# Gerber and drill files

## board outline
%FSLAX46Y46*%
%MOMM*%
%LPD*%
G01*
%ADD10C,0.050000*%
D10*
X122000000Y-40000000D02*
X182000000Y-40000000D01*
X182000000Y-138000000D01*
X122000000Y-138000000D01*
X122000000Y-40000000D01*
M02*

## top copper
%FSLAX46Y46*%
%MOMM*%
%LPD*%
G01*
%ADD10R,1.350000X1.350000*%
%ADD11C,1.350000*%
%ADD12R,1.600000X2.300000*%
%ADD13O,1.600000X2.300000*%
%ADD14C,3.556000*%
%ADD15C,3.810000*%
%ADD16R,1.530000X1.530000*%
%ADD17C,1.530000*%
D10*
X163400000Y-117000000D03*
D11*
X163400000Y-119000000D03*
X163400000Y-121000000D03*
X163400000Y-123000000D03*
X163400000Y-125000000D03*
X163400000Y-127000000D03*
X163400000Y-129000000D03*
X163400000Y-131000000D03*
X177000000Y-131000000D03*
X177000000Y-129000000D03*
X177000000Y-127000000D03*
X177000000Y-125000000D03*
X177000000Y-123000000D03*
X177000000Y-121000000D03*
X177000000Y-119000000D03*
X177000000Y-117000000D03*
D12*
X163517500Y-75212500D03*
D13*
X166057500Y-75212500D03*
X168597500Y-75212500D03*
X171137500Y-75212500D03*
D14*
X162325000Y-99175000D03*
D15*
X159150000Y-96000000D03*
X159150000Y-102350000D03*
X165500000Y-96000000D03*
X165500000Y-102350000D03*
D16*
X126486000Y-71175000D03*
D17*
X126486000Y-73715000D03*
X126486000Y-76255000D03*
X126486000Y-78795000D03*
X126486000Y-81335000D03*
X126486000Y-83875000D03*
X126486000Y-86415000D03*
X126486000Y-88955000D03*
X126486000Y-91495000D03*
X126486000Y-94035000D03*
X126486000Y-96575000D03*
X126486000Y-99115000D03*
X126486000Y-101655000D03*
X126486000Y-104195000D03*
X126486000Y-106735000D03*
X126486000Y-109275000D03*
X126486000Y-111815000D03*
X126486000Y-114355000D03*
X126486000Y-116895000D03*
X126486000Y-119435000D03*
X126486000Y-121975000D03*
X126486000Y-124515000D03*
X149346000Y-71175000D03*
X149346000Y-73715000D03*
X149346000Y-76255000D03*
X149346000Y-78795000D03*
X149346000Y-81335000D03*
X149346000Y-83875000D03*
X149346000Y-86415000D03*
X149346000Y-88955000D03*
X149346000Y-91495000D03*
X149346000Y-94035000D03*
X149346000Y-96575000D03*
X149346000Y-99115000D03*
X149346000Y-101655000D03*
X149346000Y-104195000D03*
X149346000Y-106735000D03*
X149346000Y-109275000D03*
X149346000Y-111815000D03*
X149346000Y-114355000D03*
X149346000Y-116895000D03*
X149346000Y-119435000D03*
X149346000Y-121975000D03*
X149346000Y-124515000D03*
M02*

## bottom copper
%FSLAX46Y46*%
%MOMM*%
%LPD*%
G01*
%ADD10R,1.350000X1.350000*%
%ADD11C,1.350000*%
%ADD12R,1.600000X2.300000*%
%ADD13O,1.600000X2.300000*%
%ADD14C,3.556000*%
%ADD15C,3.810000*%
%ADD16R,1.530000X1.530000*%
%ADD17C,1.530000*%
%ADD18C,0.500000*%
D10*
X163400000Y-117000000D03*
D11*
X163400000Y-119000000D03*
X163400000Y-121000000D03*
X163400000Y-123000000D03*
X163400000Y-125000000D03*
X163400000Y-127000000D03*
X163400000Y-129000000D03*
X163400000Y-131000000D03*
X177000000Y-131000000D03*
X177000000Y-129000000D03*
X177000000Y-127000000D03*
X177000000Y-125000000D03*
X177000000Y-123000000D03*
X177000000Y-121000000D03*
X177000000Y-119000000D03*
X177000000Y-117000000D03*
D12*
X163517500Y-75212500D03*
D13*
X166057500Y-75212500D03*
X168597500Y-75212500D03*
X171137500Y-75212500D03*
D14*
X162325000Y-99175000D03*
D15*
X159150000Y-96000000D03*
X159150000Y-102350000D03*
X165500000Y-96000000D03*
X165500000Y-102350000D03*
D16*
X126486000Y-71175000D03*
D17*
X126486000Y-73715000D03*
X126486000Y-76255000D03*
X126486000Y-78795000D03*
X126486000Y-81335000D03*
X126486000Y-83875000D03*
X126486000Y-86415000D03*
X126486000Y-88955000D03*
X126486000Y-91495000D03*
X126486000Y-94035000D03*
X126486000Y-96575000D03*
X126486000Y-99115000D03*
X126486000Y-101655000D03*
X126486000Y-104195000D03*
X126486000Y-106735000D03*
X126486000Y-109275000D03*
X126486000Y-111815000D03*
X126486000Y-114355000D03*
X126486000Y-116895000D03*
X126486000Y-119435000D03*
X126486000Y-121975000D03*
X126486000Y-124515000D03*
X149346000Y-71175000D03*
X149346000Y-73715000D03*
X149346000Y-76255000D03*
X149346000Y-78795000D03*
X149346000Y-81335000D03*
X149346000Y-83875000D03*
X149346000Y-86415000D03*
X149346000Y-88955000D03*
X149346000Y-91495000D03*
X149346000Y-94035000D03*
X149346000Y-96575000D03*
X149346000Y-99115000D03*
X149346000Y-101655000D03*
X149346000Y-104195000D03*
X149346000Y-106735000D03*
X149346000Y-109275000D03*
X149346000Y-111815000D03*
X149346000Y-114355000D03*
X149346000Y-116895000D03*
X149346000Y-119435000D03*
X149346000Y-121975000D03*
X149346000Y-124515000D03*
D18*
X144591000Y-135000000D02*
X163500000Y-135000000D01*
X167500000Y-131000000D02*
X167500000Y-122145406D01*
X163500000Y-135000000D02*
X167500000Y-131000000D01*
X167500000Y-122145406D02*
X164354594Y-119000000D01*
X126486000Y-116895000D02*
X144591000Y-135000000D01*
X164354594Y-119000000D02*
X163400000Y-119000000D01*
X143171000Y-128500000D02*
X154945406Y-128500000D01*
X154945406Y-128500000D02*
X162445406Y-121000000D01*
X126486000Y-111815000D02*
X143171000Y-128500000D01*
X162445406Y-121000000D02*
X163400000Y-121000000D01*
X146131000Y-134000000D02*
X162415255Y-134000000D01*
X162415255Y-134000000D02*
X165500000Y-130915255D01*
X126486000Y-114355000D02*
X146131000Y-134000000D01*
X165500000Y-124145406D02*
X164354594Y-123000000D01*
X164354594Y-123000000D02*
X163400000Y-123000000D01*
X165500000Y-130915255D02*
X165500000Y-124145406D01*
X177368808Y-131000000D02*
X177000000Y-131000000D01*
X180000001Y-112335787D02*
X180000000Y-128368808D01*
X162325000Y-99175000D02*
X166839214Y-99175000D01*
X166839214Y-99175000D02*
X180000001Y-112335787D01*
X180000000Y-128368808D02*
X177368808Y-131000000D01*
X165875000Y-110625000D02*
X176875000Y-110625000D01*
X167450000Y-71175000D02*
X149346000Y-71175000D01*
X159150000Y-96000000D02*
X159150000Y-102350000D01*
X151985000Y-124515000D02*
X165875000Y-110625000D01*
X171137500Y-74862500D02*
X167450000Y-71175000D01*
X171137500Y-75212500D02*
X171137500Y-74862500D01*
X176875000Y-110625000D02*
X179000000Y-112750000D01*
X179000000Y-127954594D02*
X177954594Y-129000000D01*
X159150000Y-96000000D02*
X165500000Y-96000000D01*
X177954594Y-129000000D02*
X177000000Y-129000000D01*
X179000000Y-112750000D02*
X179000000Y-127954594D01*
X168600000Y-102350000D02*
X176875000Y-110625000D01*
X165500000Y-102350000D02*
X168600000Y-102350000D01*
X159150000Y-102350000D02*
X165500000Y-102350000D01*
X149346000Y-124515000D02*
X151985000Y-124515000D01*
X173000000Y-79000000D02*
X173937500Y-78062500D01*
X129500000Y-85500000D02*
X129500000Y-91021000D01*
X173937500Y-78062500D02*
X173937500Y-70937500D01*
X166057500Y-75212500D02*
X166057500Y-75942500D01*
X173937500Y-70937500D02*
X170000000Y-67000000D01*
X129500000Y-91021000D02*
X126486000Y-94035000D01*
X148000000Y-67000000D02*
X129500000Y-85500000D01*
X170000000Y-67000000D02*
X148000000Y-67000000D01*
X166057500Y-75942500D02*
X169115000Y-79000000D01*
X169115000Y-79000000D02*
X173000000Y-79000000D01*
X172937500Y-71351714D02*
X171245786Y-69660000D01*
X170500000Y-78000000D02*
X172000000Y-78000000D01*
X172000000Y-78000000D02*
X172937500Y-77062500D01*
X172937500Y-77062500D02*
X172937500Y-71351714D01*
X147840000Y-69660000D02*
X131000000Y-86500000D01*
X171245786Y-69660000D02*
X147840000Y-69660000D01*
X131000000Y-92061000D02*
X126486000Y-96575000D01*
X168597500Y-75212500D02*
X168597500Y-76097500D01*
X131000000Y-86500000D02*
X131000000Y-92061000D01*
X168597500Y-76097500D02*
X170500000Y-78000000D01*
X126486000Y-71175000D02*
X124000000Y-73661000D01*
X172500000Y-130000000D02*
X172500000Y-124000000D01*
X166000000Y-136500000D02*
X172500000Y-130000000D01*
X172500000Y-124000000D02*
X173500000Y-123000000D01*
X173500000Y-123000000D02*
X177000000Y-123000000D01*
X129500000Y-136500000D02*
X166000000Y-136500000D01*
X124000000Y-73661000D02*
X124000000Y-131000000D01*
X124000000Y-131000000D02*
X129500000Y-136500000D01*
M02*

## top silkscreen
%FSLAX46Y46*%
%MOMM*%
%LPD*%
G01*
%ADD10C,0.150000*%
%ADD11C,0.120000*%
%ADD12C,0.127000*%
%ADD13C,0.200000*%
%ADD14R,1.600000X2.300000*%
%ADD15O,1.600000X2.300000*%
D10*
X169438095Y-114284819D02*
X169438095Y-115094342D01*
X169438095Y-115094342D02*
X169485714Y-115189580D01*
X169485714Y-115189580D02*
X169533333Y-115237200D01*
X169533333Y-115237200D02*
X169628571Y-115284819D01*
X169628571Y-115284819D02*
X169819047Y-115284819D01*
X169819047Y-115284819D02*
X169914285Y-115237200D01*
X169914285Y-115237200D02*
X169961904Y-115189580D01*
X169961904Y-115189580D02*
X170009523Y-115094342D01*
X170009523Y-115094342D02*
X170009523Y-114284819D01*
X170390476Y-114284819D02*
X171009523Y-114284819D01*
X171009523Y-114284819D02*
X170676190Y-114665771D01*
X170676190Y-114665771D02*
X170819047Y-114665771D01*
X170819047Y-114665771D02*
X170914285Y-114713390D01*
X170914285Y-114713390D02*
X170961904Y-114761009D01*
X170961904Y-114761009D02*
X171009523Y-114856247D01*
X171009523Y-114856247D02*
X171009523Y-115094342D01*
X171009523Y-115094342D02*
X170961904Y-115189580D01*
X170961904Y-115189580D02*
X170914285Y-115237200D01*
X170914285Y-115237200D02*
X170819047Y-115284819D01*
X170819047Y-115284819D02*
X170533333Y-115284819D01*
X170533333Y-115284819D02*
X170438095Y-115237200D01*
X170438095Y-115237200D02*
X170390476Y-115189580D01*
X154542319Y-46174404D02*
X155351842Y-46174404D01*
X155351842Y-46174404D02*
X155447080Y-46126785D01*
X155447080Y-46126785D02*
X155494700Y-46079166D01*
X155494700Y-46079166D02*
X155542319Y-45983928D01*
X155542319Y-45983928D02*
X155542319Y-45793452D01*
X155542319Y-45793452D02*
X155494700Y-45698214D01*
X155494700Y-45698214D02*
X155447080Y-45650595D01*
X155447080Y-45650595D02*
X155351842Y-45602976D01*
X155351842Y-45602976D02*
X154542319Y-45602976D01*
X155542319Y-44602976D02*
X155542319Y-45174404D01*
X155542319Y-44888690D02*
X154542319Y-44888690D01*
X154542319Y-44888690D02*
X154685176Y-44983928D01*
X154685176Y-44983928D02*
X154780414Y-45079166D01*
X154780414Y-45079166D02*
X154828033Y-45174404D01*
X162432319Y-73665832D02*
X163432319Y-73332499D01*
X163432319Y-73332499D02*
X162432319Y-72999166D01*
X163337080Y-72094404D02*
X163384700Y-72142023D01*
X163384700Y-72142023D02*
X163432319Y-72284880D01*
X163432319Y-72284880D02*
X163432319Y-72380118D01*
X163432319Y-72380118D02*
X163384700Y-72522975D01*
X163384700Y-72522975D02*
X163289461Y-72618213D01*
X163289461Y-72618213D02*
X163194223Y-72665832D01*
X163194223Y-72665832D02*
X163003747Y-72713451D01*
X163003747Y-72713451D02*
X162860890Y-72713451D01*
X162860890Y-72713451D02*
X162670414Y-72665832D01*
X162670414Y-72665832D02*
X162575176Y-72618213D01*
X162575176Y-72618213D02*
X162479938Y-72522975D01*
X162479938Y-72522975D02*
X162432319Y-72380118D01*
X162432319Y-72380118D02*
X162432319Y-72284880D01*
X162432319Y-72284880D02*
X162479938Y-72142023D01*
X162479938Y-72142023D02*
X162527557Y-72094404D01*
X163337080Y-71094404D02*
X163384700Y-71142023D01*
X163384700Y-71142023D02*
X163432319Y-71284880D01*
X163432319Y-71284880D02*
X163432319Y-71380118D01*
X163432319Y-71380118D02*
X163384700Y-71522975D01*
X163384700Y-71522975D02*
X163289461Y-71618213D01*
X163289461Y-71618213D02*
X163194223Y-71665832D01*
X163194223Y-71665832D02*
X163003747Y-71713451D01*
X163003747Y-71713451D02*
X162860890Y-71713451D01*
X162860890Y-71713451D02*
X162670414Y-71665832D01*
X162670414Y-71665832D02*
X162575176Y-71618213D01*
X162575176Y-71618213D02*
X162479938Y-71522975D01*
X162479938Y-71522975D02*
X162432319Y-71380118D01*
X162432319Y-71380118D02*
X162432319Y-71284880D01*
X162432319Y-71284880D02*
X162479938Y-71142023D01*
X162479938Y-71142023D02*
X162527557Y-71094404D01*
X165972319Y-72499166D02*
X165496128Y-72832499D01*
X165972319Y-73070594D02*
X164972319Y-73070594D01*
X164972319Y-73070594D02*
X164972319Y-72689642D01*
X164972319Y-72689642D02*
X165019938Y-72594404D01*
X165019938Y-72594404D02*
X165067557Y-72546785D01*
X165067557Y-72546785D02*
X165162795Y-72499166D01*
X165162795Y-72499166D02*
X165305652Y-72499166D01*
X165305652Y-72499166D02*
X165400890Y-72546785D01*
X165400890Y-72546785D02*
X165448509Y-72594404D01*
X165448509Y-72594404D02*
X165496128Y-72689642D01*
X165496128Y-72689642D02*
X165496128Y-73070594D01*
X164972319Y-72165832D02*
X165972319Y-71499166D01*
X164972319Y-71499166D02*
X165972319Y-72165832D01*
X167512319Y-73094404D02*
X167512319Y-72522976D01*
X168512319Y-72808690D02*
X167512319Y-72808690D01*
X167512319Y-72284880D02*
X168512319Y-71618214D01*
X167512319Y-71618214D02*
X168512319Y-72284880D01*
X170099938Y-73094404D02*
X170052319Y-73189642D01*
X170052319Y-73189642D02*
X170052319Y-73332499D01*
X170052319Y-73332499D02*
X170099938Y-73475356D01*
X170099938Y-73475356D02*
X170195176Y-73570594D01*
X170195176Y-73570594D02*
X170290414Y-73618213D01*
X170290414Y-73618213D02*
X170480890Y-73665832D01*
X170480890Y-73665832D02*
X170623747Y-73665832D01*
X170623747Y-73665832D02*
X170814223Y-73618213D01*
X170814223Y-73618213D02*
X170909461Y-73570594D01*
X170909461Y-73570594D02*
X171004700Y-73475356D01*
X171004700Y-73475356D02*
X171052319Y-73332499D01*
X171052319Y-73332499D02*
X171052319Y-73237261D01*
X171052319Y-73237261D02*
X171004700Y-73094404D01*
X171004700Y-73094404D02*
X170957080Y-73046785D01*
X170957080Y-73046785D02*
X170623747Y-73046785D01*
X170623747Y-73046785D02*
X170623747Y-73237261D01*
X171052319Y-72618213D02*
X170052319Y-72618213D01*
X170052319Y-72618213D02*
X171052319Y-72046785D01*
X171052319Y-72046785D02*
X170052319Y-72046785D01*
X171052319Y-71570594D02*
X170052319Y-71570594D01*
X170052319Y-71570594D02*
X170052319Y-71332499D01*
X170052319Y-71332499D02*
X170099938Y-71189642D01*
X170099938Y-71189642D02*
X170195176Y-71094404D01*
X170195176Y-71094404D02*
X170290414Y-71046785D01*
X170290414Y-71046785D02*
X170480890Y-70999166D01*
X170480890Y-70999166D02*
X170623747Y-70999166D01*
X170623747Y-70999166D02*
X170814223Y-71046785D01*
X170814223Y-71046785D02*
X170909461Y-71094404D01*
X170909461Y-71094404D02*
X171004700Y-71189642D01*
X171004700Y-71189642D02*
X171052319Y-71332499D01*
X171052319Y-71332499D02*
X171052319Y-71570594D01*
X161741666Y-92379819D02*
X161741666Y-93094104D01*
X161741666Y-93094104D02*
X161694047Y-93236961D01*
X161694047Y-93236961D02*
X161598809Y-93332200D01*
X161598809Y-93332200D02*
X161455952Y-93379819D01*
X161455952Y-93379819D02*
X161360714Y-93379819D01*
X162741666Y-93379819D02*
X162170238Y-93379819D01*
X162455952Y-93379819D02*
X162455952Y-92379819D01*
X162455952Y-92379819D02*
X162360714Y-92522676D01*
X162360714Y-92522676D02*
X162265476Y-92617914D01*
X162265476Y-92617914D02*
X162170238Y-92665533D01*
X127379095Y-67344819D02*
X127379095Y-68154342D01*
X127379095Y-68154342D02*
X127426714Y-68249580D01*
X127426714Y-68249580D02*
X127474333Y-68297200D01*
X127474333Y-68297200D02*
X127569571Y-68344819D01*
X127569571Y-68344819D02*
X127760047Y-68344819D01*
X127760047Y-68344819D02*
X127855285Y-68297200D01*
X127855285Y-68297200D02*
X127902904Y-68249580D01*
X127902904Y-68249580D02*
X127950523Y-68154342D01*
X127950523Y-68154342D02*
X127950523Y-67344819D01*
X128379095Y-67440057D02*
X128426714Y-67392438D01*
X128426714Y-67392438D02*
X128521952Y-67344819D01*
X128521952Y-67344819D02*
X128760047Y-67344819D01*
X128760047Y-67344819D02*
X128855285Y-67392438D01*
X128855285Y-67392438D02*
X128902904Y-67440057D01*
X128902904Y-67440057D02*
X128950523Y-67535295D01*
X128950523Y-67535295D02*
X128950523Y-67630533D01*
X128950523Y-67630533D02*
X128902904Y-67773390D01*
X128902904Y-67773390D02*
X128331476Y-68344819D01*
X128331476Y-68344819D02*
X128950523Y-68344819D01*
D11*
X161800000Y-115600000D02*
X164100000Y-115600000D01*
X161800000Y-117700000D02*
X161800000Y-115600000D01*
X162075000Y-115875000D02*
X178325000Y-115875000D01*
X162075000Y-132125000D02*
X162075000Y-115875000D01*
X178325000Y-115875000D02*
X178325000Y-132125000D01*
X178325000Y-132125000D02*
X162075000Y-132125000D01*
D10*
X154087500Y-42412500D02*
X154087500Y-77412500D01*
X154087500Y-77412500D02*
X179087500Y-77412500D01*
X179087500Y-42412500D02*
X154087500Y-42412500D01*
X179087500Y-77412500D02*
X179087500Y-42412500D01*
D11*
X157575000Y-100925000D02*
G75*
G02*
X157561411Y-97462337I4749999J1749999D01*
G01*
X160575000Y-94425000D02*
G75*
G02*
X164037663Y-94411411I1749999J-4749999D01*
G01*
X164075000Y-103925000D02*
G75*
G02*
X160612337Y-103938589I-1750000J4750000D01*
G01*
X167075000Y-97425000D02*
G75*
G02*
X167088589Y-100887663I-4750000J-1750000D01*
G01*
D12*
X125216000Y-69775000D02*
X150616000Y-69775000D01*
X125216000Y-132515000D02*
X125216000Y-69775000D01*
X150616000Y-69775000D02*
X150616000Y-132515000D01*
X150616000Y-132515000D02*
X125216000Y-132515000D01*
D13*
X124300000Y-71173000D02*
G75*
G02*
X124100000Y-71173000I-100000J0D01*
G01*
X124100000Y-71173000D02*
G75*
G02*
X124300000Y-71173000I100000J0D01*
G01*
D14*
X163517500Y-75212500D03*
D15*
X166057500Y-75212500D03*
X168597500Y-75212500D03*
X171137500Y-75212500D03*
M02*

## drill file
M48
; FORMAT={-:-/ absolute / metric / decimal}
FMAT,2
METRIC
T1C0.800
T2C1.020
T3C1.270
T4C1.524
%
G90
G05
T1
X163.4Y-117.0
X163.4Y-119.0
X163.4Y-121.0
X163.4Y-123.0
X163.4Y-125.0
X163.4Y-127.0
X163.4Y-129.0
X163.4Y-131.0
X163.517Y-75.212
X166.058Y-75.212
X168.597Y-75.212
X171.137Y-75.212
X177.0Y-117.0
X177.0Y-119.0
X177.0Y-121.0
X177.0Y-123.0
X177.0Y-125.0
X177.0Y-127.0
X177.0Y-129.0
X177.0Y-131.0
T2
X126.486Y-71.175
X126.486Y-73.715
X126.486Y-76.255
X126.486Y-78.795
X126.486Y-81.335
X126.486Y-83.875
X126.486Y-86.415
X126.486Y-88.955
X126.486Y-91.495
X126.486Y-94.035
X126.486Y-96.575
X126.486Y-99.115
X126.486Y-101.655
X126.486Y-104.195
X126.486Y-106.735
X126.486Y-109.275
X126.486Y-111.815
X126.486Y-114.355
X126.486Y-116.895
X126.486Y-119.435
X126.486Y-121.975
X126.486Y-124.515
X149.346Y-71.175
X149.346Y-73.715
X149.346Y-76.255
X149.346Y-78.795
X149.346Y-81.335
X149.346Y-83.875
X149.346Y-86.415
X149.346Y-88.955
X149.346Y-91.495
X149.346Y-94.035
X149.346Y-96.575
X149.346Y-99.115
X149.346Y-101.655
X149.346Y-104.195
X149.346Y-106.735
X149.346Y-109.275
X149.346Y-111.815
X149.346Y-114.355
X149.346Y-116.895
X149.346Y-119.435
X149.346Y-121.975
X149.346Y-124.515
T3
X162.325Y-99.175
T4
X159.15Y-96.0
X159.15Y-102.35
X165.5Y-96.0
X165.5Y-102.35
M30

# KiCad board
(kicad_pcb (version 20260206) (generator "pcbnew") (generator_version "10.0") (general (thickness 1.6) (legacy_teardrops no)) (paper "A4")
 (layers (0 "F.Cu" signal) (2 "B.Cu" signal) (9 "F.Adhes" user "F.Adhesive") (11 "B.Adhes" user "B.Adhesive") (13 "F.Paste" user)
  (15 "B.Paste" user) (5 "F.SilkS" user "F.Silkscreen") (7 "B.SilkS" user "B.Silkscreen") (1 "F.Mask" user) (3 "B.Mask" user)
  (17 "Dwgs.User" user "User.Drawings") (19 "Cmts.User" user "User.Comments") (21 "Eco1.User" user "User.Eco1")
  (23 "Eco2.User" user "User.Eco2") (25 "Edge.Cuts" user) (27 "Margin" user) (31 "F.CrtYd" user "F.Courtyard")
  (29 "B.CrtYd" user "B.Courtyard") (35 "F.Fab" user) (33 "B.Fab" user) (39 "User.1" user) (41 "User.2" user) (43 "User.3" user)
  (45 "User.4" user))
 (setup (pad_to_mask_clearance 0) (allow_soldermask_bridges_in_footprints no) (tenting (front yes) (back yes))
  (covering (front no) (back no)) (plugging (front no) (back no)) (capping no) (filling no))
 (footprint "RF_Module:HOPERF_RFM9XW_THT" (layer "F.Cu") (at 163.4 117)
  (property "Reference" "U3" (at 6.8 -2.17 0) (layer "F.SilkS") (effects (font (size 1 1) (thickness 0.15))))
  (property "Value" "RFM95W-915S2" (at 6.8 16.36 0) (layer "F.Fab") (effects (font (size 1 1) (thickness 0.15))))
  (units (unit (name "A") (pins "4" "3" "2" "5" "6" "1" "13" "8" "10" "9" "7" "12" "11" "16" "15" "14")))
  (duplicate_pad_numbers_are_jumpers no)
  (fp_line (start -1.6 -1.4) (end 0.7 -1.4) (stroke (width 0.12) (type solid)) (layer "F.SilkS"))
  (fp_line (start -1.6 0.7) (end -1.6 -1.4) (stroke (width 0.12) (type solid)) (layer "F.SilkS"))
  (fp_line (start -1.325 -1.125) (end 14.925 -1.125) (stroke (width 0.12) (type solid)) (layer "F.SilkS"))
  (fp_line (start -1.325 15.125) (end -1.325 -1.125) (stroke (width 0.12) (type solid)) (layer "F.SilkS"))
  (fp_line (start 14.925 -1.125) (end 14.925 15.125) (stroke (width 0.12) (type solid)) (layer "F.SilkS"))
  (fp_line (start 14.925 15.125) (end -1.325 15.125) (stroke (width 0.12) (type solid)) (layer "F.SilkS"))
  (pad "1" thru_hole rect (at 0 0) (size 1.35 1.35) (drill 0.8) (layers "*.Cu" "*.Mask") (remove_unused_layers no)
   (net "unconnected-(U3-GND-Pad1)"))
  (pad "2" thru_hole circle (at 0 2) (size 1.35 1.35) (drill 0.8) (layers "*.Cu" "*.Mask") (remove_unused_layers no) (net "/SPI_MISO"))
  (pad "3" thru_hole circle (at 0 4) (size 1.35 1.35) (drill 0.8) (layers "*.Cu" "*.Mask") (remove_unused_layers no) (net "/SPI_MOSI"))
  (pad "4" thru_hole circle (at 0 6) (size 1.35 1.35) (drill 0.8) (layers "*.Cu" "*.Mask") (remove_unused_layers no) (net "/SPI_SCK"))
  (pad "5" thru_hole circle (at 0 8) (size 1.35 1.35) (drill 0.8) (layers "*.Cu" "*.Mask") (remove_unused_layers no) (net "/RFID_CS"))
  (pad "6" thru_hole circle (at 0 10) (size 1.35 1.35) (drill 0.8) (layers "*.Cu" "*.Mask") (remove_unused_layers no) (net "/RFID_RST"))
  (pad "7" thru_hole circle (at 0 12) (size 1.35 1.35) (drill 0.8) (layers "*.Cu" "*.Mask") (remove_unused_layers no)
   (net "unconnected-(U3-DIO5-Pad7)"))
  (pad "8" thru_hole circle (at 0 14) (size 1.35 1.35) (drill 0.8) (layers "*.Cu" "*.Mask") (remove_unused_layers no)
   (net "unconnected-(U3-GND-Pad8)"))
  (pad "9" thru_hole circle (at 13.6 14) (size 1.35 1.35) (drill 0.8) (layers "*.Cu" "*.Mask") (remove_unused_layers no) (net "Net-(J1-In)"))
  (pad "10" thru_hole circle (at 13.6 12) (size 1.35 1.35) (drill 0.8) (layers "*.Cu" "*.Mask") (remove_unused_layers no)
   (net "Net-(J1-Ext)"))
  (pad "11" thru_hole circle (at 13.6 10) (size 1.35 1.35) (drill 0.8) (layers "*.Cu" "*.Mask") (remove_unused_layers no)
   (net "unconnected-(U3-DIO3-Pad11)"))
  (pad "12" thru_hole circle (at 13.6 8) (size 1.35 1.35) (drill 0.8) (layers "*.Cu" "*.Mask") (remove_unused_layers no)
   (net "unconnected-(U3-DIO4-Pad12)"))
  (pad "13" thru_hole circle (at 13.6 6) (size 1.35 1.35) (drill 0.8) (layers "*.Cu" "*.Mask") (remove_unused_layers no)
   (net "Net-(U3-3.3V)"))
  (pad "14" thru_hole circle (at 13.6 4) (size 1.35 1.35) (drill 0.8) (layers "*.Cu" "*.Mask") (remove_unused_layers no)
   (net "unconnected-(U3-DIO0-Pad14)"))
  (pad "15" thru_hole circle (at 13.6 2) (size 1.35 1.35) (drill 0.8) (layers "*.Cu" "*.Mask") (remove_unused_layers no)
   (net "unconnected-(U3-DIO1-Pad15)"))
  (pad "16" thru_hole circle (at 13.6 0) (size 1.35 1.35) (drill 0.8) (layers "*.Cu" "*.Mask") (remove_unused_layers no)
   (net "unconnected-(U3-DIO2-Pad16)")))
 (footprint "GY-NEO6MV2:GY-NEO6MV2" (layer "F.Cu") (at 154.0875 77.4125 -90)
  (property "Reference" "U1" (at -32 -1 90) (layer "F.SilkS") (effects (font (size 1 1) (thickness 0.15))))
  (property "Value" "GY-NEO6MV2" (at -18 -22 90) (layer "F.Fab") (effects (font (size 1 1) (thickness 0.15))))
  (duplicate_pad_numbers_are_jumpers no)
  (fp_line (start -35 0) (end 0 0) (stroke (width 0.15) (type solid)) (layer "F.SilkS"))
  (fp_line (start 0 0) (end 0 -25) (stroke (width 0.15) (type solid)) (layer "F.SilkS"))
  (fp_line (start -35 -25) (end -35 0) (stroke (width 0.15) (type solid)) (layer "F.SilkS"))
  (fp_line (start 0 -25) (end -35 -25) (stroke (width 0.15) (type solid)) (layer "F.SilkS"))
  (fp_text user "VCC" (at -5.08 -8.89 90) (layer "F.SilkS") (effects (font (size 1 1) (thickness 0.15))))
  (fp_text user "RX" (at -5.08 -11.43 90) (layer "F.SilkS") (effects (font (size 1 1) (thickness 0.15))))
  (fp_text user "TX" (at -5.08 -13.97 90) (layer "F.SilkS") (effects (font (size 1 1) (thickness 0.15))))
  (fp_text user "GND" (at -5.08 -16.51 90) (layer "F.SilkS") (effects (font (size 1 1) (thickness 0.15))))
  (pad "1" thru_hole rect (at -2.2 -9.43 270) (size 2.3 1.6) (drill 0.8) (layers "*.Cu" "*.Mask" "F.SilkS") (remove_unused_layers no)
   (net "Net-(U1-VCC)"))
  (pad "2" thru_hole oval (at -2.2 -11.97 270) (size 2.3 1.6) (drill 0.8) (layers "*.Cu" "*.Mask" "F.SilkS") (remove_unused_layers no)
   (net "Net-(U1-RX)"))
  (pad "3" thru_hole oval (at -2.2 -14.51 270) (size 2.3 1.6) (drill 0.8) (layers "*.Cu" "*.Mask" "F.SilkS") (remove_unused_layers no)
   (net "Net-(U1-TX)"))
  (pad "4" thru_hole oval (at -2.2 -17.05 270) (size 2.3 1.6) (drill 0.8) (layers "*.Cu" "*.Mask" "F.SilkS") (remove_unused_layers no)
   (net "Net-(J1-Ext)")))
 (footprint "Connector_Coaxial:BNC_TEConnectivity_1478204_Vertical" (layer "F.Cu") (at 162.325 99.175)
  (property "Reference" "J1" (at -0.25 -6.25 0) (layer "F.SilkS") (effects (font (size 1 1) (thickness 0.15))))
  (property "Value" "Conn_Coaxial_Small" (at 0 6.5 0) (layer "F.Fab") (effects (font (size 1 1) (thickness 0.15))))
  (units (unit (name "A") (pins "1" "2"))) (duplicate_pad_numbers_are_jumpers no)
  (fp_arc (start -4.75 1.75) (mid -5.062075 0.019867) (end -4.763589 -1.712663) (stroke (width 0.12) (type solid)) (layer "F.SilkS"))
  (fp_arc (start -1.75 -4.75) (mid -0.019867 -5.062075) (end 1.712663 -4.763589) (stroke (width 0.12) (type solid)) (layer "F.SilkS"))
  (fp_arc (start 1.75 4.75) (mid 0.019867 5.062075) (end -1.712663 4.763589) (stroke (width 0.12) (type solid)) (layer "F.SilkS"))
  (fp_arc (start 4.75 -1.75) (mid 5.062075 -0.019867) (end 4.763589 1.712663) (stroke (width 0.12) (type solid)) (layer "F.SilkS"))
  (pad "1" thru_hole circle (at 0 0) (size 3.556 3.556) (drill 1.27) (layers "*.Cu" "*.Mask") (remove_unused_layers no) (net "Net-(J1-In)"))
  (pad "2" thru_hole circle (at -3.175 -3.175) (size 3.81 3.81) (drill 1.524) (layers "*.Cu" "*.Mask") (remove_unused_layers no)
   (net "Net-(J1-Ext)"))
  (pad "2" thru_hole circle (at -3.175 3.175) (size 3.81 3.81) (drill 1.524) (layers "*.Cu" "*.Mask") (remove_unused_layers no)
   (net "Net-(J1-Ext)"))
  (pad "2" thru_hole circle (at 3.175 -3.175) (size 3.81 3.81) (drill 1.524) (layers "*.Cu" "*.Mask") (remove_unused_layers no)
   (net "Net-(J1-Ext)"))
  (pad "2" thru_hole circle (at 3.175 3.175) (size 3.81 3.81) (drill 1.524) (layers "*.Cu" "*.Mask") (remove_unused_layers no)
   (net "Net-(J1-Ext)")))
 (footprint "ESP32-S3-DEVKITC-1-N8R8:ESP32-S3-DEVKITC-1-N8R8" (layer "F.Cu") (at 137.916 101.145)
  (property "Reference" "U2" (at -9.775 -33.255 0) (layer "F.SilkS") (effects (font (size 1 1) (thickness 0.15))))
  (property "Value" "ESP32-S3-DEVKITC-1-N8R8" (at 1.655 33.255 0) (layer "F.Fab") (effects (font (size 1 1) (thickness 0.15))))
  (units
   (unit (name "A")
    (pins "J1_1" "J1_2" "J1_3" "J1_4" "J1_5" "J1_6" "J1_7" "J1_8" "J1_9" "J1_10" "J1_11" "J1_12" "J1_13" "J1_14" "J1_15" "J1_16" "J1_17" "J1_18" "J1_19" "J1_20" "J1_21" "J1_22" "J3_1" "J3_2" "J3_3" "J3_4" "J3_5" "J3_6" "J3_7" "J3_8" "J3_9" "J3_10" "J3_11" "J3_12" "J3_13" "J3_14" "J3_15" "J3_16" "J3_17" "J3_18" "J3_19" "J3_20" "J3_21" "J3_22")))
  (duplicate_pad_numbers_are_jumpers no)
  (fp_line (start -12.7 -31.37) (end 12.7 -31.37) (stroke (width 0.127) (type solid)) (layer "F.SilkS"))
  (fp_line (start -12.7 31.37) (end -12.7 -31.37) (stroke (width 0.127) (type solid)) (layer "F.SilkS"))
  (fp_line (start 12.7 -31.37) (end 12.7 31.37) (stroke (width 0.127) (type solid)) (layer "F.SilkS"))
  (fp_line (start 12.7 31.37) (end -12.7 31.37) (stroke (width 0.127) (type solid)) (layer "F.SilkS"))
  (fp_circle (center -13.716 -29.972) (end -13.616 -29.972) (stroke (width 0.2) (type solid)) (fill no) (layer "F.SilkS"))
  (pad "J1_1" thru_hole rect (at -11.43 -29.97) (size 1.53 1.53) (drill 1.02) (layers "*.Cu" "*.Mask") (remove_unused_layers no)
   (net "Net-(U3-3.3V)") (solder_mask_margin 0.102))
  (pad "J1_2" thru_hole circle (at -11.43 -27.43) (size 1.53 1.53) (drill 1.02) (layers "*.Cu" "*.Mask") (remove_unused_layers no)
   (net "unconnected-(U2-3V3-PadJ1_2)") (solder_mask_margin 0.102))
  (pad "J1_3" thru_hole circle (at -11.43 -24.89) (size 1.53 1.53) (drill 1.02) (layers "*.Cu" "*.Mask") (remove_unused_layers no)
   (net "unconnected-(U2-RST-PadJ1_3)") (solder_mask_margin 0.102))
  (pad "J1_4" thru_hole circle (at -11.43 -22.35) (size 1.53 1.53) (drill 1.02) (layers "*.Cu" "*.Mask") (remove_unused_layers no)
   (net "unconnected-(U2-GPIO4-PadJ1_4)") (solder_mask_margin 0.102))
  (pad "J1_5" thru_hole circle (at -11.43 -19.81) (size 1.53 1.53) (drill 1.02) (layers "*.Cu" "*.Mask") (remove_unused_layers no)
   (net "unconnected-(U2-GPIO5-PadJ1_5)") (solder_mask_margin 0.102))
  (pad "J1_6" thru_hole circle (at -11.43 -17.27) (size 1.53 1.53) (drill 1.02) (layers "*.Cu" "*.Mask") (remove_unused_layers no)
   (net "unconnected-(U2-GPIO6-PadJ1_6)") (solder_mask_margin 0.102))
  (pad "J1_7" thru_hole circle (at -11.43 -14.73) (size 1.53 1.53) (drill 1.02) (layers "*.Cu" "*.Mask") (remove_unused_layers no)
   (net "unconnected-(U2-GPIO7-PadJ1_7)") (solder_mask_margin 0.102))
  (pad "J1_8" thru_hole circle (at -11.43 -12.19) (size 1.53 1.53) (drill 1.02) (layers "*.Cu" "*.Mask") (remove_unused_layers no)
   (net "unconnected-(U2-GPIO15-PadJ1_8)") (solder_mask_margin 0.102))
  (pad "J1_9" thru_hole circle (at -11.43 -9.65) (size 1.53 1.53) (drill 1.02) (layers "*.Cu" "*.Mask") (remove_unused_layers no)
   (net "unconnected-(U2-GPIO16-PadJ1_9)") (solder_mask_margin 0.102))
  (pad "J1_10" thru_hole circle (at -11.43 -7.11) (size 1.53 1.53) (drill 1.02) (layers "*.Cu" "*.Mask") (remove_unused_layers no)
   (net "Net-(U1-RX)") (solder_mask_margin 0.102))
  (pad "J1_11" thru_hole circle (at -11.43 -4.57) (size 1.53 1.53) (drill 1.02) (layers "*.Cu" "*.Mask") (remove_unused_layers no)
   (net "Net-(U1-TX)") (solder_mask_margin 0.102))
  (pad "J1_12" thru_hole circle (at -11.43 -2.03) (size 1.53 1.53) (drill 1.02) (layers "*.Cu" "*.Mask") (remove_unused_layers no)
   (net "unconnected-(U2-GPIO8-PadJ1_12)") (solder_mask_margin 0.102))
  (pad "J1_13" thru_hole circle (at -11.43 0.51) (size 1.53 1.53) (drill 1.02) (layers "*.Cu" "*.Mask") (remove_unused_layers no)
   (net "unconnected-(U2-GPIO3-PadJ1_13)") (solder_mask_margin 0.102))
  (pad "J1_14" thru_hole circle (at -11.43 3.05) (size 1.53 1.53) (drill 1.02) (layers "*.Cu" "*.Mask") (remove_unused_layers no)
   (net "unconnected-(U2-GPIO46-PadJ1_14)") (solder_mask_margin 0.102))
  (pad "J1_15" thru_hole circle (at -11.43 5.59) (size 1.53 1.53) (drill 1.02) (layers "*.Cu" "*.Mask") (remove_unused_layers no)
   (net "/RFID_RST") (solder_mask_margin 0.102))
  (pad "J1_16" thru_hole circle (at -11.43 8.13) (size 1.53 1.53) (drill 1.02) (layers "*.Cu" "*.Mask") (remove_unused_layers no)
   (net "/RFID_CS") (solder_mask_margin 0.102))
  (pad "J1_17" thru_hole circle (at -11.43 10.67) (size 1.53 1.53) (drill 1.02) (layers "*.Cu" "*.Mask") (remove_unused_layers no)
   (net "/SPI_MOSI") (solder_mask_margin 0.102))
  (pad "J1_18" thru_hole circle (at -11.43 13.21) (size 1.53 1.53) (drill 1.02) (layers "*.Cu" "*.Mask") (remove_unused_layers no)
   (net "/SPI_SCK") (solder_mask_margin 0.102))
  (pad "J1_19" thru_hole circle (at -11.43 15.75) (size 1.53 1.53) (drill 1.02) (layers "*.Cu" "*.Mask") (remove_unused_layers no)
   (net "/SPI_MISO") (solder_mask_margin 0.102))
  (pad "J1_20" thru_hole circle (at -11.43 18.29) (size 1.53 1.53) (drill 1.02) (layers "*.Cu" "*.Mask") (remove_unused_layers no)
   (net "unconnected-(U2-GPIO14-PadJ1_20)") (solder_mask_margin 0.102))
  (pad "J1_21" thru_hole circle (at -11.43 20.83) (size 1.53 1.53) (drill 1.02) (layers "*.Cu" "*.Mask") (remove_unused_layers no)
   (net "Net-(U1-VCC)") (solder_mask_margin 0.102))
  (pad "J1_22" thru_hole circle (at -11.43 23.37) (size 1.53 1.53) (drill 1.02) (layers "*.Cu" "*.Mask") (remove_unused_layers no)
   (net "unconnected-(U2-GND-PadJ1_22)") (solder_mask_margin 0.102))
  (pad "J3_1" thru_hole circle (at 11.43 -29.97) (size 1.53 1.53) (drill 1.02) (layers "*.Cu" "*.Mask") (remove_unused_layers no)
   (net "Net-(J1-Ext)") (solder_mask_margin 0.102))
  (pad "J3_2" thru_hole circle (at 11.43 -27.43) (size 1.53 1.53) (drill 1.02) (layers "*.Cu" "*.Mask") (remove_unused_layers no)
   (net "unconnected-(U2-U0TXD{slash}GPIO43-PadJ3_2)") (solder_mask_margin 0.102))
  (pad "J3_3" thru_hole circle (at 11.43 -24.89) (size 1.53 1.53) (drill 1.02) (layers "*.Cu" "*.Mask") (remove_unused_layers no)
   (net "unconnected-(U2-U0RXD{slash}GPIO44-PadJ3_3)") (solder_mask_margin 0.102))
  (pad "J3_4" thru_hole circle (at 11.43 -22.35) (size 1.53 1.53) (drill 1.02) (layers "*.Cu" "*.Mask") (remove_unused_layers no)
   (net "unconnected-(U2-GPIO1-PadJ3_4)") (solder_mask_margin 0.102))
  (pad "J3_5" thru_hole circle (at 11.43 -19.81) (size 1.53 1.53) (drill 1.02) (layers "*.Cu" "*.Mask") (remove_unused_layers no)
   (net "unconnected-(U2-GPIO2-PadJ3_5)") (solder_mask_margin 0.102))
  (pad "J3_6" thru_hole circle (at 11.43 -17.27) (size 1.53 1.53) (drill 1.02) (layers "*.Cu" "*.Mask") (remove_unused_layers no)
   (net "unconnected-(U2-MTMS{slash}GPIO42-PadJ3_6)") (solder_mask_margin 0.102))
  (pad "J3_7" thru_hole circle (at 11.43 -14.73) (size 1.53 1.53) (drill 1.02) (layers "*.Cu" "*.Mask") (remove_unused_layers no)
   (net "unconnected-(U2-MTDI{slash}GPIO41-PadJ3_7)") (solder_mask_margin 0.102))
  (pad "J3_8" thru_hole circle (at 11.43 -12.19) (size 1.53 1.53) (drill 1.02) (layers "*.Cu" "*.Mask") (remove_unused_layers no)
   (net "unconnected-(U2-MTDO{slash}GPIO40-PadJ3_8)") (solder_mask_margin 0.102))
  (pad "J3_9" thru_hole circle (at 11.43 -9.65) (size 1.53 1.53) (drill 1.02) (layers "*.Cu" "*.Mask") (remove_unused_layers no)
   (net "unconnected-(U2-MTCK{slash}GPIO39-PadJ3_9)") (solder_mask_margin 0.102))
  (pad "J3_10" thru_hole circle (at 11.43 -7.11) (size 1.53 1.53) (drill 1.02) (layers "*.Cu" "*.Mask") (remove_unused_layers no)
   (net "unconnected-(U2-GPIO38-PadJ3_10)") (solder_mask_margin 0.102))
  (pad "J3_11" thru_hole circle (at 11.43 -4.57) (size 1.53 1.53) (drill 1.02) (layers "*.Cu" "*.Mask") (remove_unused_layers no)
   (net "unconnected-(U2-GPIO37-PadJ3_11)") (solder_mask_margin 0.102))
  (pad "J3_12" thru_hole circle (at 11.43 -2.03) (size 1.53 1.53) (drill 1.02) (layers "*.Cu" "*.Mask") (remove_unused_layers no)
   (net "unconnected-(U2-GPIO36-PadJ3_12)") (solder_mask_margin 0.102))
  (pad "J3_13" thru_hole circle (at 11.43 0.51) (size 1.53 1.53) (drill 1.02) (layers "*.Cu" "*.Mask") (remove_unused_layers no)
   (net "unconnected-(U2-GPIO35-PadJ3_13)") (solder_mask_margin 0.102))
  (pad "J3_14" thru_hole circle (at 11.43 3.05) (size 1.53 1.53) (drill 1.02) (layers "*.Cu" "*.Mask") (remove_unused_layers no)
   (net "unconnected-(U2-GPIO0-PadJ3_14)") (solder_mask_margin 0.102))
  (pad "J3_15" thru_hole circle (at 11.43 5.59) (size 1.53 1.53) (drill 1.02) (layers "*.Cu" "*.Mask") (remove_unused_layers no)
   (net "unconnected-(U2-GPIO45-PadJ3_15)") (solder_mask_margin 0.102))
  (pad "J3_16" thru_hole circle (at 11.43 8.13) (size 1.53 1.53) (drill 1.02) (layers "*.Cu" "*.Mask") (remove_unused_layers no)
   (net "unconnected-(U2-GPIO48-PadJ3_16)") (solder_mask_margin 0.102))
  (pad "J3_17" thru_hole circle (at 11.43 10.67) (size 1.53 1.53) (drill 1.02) (layers "*.Cu" "*.Mask") (remove_unused_layers no)
   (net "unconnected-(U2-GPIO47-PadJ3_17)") (solder_mask_margin 0.102))
  (pad "J3_18" thru_hole circle (at 11.43 13.21) (size 1.53 1.53) (drill 1.02) (layers "*.Cu" "*.Mask") (remove_unused_layers no)
   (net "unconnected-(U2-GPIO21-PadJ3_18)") (solder_mask_margin 0.102))
  (pad "J3_19" thru_hole circle (at 11.43 15.75) (size 1.53 1.53) (drill 1.02) (layers "*.Cu" "*.Mask") (remove_unused_layers no)
   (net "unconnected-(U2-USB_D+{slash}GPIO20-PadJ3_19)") (solder_mask_margin 0.102))
  (pad "J3_20" thru_hole circle (at 11.43 18.29) (size 1.53 1.53) (drill 1.02) (layers "*.Cu" "*.Mask") (remove_unused_layers no)
   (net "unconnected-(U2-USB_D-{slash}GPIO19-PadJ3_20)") (solder_mask_margin 0.102))
  (pad "J3_21" thru_hole circle (at 11.43 20.83) (size 1.53 1.53) (drill 1.02) (layers "*.Cu" "*.Mask") (remove_unused_layers no)
   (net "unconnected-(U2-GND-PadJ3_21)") (solder_mask_margin 0.102))
  (pad "J3_22" thru_hole circle (at 11.43 23.37) (size 1.53 1.53) (drill 1.02) (layers "*.Cu" "*.Mask") (remove_unused_layers no)
   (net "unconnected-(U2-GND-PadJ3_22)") (solder_mask_margin 0.102)))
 (gr_rect (start 122 40) (end 182 138) (stroke (width 0.05) (type solid)) (fill no) (layer "Edge.Cuts"))
 (segment (start 144.591 135) (end 163.5 135) (width 0.5) (layer "B.Cu") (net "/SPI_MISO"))
 (segment (start 167.5 131) (end 167.5 122.145406) (width 0.5) (layer "B.Cu") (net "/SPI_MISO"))
 (segment (start 163.5 135) (end 167.5 131) (width 0.5) (layer "B.Cu") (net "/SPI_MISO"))
 (segment (start 167.5 122.145406) (end 164.354594 119) (width 0.5) (layer "B.Cu") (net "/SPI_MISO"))
 (segment (start 126.486 116.895) (end 144.591 135) (width 0.5) (layer "B.Cu") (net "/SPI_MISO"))
 (segment (start 164.354594 119) (end 163.4 119) (width 0.5) (layer "B.Cu") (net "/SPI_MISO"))
 (segment (start 143.171 128.5) (end 154.945406 128.5) (width 0.5) (layer "B.Cu") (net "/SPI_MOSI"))
 (segment (start 154.945406 128.5) (end 162.445406 121) (width 0.5) (layer "B.Cu") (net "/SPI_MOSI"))
 (segment (start 126.486 111.815) (end 143.171 128.5) (width 0.5) (layer "B.Cu") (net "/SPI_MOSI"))
 (segment (start 162.445406 121) (end 163.4 121) (width 0.5) (layer "B.Cu") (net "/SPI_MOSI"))
 (segment (start 146.131 134) (end 162.415255 134) (width 0.5) (layer "B.Cu") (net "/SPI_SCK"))
 (segment (start 162.415255 134) (end 165.5 130.915255) (width 0.5) (layer "B.Cu") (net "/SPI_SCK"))
 (segment (start 126.486 114.355) (end 146.131 134) (width 0.5) (layer "B.Cu") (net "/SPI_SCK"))
 (segment (start 165.5 124.145406) (end 164.354594 123) (width 0.5) (layer "B.Cu") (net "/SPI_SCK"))
 (segment (start 164.354594 123) (end 163.4 123) (width 0.5) (layer "B.Cu") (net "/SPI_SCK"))
 (segment (start 165.5 130.915255) (end 165.5 124.145406) (width 0.5) (layer "B.Cu") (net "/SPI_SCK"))
 (segment (start 177.368808 131) (end 177 131) (width 0.5) (layer "B.Cu") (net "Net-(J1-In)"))
 (segment (start 180.000001 112.335787) (end 180 128.368808) (width 0.5) (layer "B.Cu") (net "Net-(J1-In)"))
 (segment (start 162.325 99.175) (end 166.839214 99.175) (width 0.5) (layer "B.Cu") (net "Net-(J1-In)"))
 (segment (start 166.839214 99.175) (end 180.000001 112.335787) (width 0.5) (layer "B.Cu") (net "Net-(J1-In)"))
 (segment (start 180 128.368808) (end 177.368808 131) (width 0.5) (layer "B.Cu") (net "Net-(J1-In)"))
 (segment (start 165.875 110.625) (end 176.875 110.625) (width 0.5) (layer "B.Cu") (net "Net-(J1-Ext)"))
 (segment (start 167.45 71.175) (end 149.346 71.175) (width 0.5) (layer "B.Cu") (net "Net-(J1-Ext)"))
 (segment (start 159.15 96) (end 159.15 102.35) (width 0.5) (layer "B.Cu") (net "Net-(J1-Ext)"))
 (segment (start 151.985 124.515) (end 165.875 110.625) (width 0.5) (layer "B.Cu") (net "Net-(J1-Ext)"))
 (segment (start 171.1375 74.8625) (end 167.45 71.175) (width 0.5) (layer "B.Cu") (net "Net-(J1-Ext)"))
 (segment (start 171.1375 75.2125) (end 171.1375 74.8625) (width 0.5) (layer "B.Cu") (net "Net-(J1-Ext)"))
 (segment (start 176.875 110.625) (end 179 112.75) (width 0.5) (layer "B.Cu") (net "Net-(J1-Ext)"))
 (segment (start 179 127.954594) (end 177.954594 129) (width 0.5) (layer "B.Cu") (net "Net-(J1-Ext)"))
 (segment (start 159.15 96) (end 165.5 96) (width 0.5) (layer "B.Cu") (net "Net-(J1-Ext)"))
 (segment (start 177.954594 129) (end 177 129) (width 0.5) (layer "B.Cu") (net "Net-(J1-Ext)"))
 (segment (start 179 112.75) (end 179 127.954594) (width 0.5) (layer "B.Cu") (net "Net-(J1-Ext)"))
 (segment (start 168.6 102.35) (end 176.875 110.625) (width 0.5) (layer "B.Cu") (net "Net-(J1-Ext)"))
 (segment (start 165.5 102.35) (end 168.6 102.35) (width 0.5) (layer "B.Cu") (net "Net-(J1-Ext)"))
 (segment (start 159.15 102.35) (end 165.5 102.35) (width 0.5) (layer "B.Cu") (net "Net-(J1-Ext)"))
 (segment (start 149.346 124.515) (end 151.985 124.515) (width 0.5) (layer "B.Cu") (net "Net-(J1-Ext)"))
 (segment (start 173 79) (end 173.9375 78.0625) (width 0.5) (layer "B.Cu") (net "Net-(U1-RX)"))
 (segment (start 129.5 85.5) (end 129.5 91.021) (width 0.5) (layer "B.Cu") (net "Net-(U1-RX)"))
 (segment (start 173.9375 78.0625) (end 173.9375 70.9375) (width 0.5) (layer "B.Cu") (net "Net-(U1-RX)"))
 (segment (start 166.0575 75.2125) (end 166.0575 75.9425) (width 0.5) (layer "B.Cu") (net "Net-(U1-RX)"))
 (segment (start 173.9375 70.9375) (end 170 67) (width 0.5) (layer "B.Cu") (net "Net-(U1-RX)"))
 (segment (start 129.5 91.021) (end 126.486 94.035) (width 0.5) (layer "B.Cu") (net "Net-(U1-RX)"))
 (segment (start 148 67) (end 129.5 85.5) (width 0.5) (layer "B.Cu") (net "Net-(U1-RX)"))
 (segment (start 170 67) (end 148 67) (width 0.5) (layer "B.Cu") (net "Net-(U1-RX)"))
 (segment (start 166.0575 75.9425) (end 169.115 79) (width 0.5) (layer "B.Cu") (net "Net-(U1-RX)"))
 (segment (start 169.115 79) (end 173 79) (width 0.5) (layer "B.Cu") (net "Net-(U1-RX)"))
 (segment (start 172.9375 71.351714) (end 171.245786 69.66) (width 0.5) (layer "B.Cu") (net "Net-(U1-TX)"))
 (segment (start 170.5 78) (end 172 78) (width 0.5) (layer "B.Cu") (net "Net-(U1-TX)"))
 (segment (start 172 78) (end 172.9375 77.0625) (width 0.5) (layer "B.Cu") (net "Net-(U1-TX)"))
 (segment (start 172.9375 77.0625) (end 172.9375 71.351714) (width 0.5) (layer "B.Cu") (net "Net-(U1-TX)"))
 (segment (start 147.84 69.66) (end 131 86.5) (width 0.5) (layer "B.Cu") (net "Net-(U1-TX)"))
 (segment (start 171.245786 69.66) (end 147.84 69.66) (width 0.5) (layer "B.Cu") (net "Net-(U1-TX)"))
 (segment (start 131 92.061) (end 126.486 96.575) (width 0.5) (layer "B.Cu") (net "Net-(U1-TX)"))
 (segment (start 168.5975 75.2125) (end 168.5975 76.0975) (width 0.5) (layer "B.Cu") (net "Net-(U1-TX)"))
 (segment (start 131 86.5) (end 131 92.061) (width 0.5) (layer "B.Cu") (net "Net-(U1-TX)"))
 (segment (start 168.5975 76.0975) (end 170.5 78) (width 0.5) (layer "B.Cu") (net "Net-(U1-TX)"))
 (segment (start 126.486 71.175) (end 124 73.661) (width 0.5) (layer "B.Cu") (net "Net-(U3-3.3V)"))
 (segment (start 172.5 130) (end 172.5 124) (width 0.5) (layer "B.Cu") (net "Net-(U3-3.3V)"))
 (segment (start 166 136.5) (end 172.5 130) (width 0.5) (layer "B.Cu") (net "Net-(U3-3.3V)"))
 (segment (start 172.5 124) (end 173.5 123) (width 0.5) (layer "B.Cu") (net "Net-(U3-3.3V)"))
 (segment (start 173.5 123) (end 177 123) (width 0.5) (layer "B.Cu") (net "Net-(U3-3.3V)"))
 (segment (start 129.5 136.5) (end 166 136.5) (width 0.5) (layer "B.Cu") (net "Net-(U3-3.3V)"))
 (segment (start 124 73.661) (end 124 131) (width 0.5) (layer "B.Cu") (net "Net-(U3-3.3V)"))
 (segment (start 124 131) (end 129.5 136.5) (width 0.5) (layer "B.Cu") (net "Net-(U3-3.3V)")))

